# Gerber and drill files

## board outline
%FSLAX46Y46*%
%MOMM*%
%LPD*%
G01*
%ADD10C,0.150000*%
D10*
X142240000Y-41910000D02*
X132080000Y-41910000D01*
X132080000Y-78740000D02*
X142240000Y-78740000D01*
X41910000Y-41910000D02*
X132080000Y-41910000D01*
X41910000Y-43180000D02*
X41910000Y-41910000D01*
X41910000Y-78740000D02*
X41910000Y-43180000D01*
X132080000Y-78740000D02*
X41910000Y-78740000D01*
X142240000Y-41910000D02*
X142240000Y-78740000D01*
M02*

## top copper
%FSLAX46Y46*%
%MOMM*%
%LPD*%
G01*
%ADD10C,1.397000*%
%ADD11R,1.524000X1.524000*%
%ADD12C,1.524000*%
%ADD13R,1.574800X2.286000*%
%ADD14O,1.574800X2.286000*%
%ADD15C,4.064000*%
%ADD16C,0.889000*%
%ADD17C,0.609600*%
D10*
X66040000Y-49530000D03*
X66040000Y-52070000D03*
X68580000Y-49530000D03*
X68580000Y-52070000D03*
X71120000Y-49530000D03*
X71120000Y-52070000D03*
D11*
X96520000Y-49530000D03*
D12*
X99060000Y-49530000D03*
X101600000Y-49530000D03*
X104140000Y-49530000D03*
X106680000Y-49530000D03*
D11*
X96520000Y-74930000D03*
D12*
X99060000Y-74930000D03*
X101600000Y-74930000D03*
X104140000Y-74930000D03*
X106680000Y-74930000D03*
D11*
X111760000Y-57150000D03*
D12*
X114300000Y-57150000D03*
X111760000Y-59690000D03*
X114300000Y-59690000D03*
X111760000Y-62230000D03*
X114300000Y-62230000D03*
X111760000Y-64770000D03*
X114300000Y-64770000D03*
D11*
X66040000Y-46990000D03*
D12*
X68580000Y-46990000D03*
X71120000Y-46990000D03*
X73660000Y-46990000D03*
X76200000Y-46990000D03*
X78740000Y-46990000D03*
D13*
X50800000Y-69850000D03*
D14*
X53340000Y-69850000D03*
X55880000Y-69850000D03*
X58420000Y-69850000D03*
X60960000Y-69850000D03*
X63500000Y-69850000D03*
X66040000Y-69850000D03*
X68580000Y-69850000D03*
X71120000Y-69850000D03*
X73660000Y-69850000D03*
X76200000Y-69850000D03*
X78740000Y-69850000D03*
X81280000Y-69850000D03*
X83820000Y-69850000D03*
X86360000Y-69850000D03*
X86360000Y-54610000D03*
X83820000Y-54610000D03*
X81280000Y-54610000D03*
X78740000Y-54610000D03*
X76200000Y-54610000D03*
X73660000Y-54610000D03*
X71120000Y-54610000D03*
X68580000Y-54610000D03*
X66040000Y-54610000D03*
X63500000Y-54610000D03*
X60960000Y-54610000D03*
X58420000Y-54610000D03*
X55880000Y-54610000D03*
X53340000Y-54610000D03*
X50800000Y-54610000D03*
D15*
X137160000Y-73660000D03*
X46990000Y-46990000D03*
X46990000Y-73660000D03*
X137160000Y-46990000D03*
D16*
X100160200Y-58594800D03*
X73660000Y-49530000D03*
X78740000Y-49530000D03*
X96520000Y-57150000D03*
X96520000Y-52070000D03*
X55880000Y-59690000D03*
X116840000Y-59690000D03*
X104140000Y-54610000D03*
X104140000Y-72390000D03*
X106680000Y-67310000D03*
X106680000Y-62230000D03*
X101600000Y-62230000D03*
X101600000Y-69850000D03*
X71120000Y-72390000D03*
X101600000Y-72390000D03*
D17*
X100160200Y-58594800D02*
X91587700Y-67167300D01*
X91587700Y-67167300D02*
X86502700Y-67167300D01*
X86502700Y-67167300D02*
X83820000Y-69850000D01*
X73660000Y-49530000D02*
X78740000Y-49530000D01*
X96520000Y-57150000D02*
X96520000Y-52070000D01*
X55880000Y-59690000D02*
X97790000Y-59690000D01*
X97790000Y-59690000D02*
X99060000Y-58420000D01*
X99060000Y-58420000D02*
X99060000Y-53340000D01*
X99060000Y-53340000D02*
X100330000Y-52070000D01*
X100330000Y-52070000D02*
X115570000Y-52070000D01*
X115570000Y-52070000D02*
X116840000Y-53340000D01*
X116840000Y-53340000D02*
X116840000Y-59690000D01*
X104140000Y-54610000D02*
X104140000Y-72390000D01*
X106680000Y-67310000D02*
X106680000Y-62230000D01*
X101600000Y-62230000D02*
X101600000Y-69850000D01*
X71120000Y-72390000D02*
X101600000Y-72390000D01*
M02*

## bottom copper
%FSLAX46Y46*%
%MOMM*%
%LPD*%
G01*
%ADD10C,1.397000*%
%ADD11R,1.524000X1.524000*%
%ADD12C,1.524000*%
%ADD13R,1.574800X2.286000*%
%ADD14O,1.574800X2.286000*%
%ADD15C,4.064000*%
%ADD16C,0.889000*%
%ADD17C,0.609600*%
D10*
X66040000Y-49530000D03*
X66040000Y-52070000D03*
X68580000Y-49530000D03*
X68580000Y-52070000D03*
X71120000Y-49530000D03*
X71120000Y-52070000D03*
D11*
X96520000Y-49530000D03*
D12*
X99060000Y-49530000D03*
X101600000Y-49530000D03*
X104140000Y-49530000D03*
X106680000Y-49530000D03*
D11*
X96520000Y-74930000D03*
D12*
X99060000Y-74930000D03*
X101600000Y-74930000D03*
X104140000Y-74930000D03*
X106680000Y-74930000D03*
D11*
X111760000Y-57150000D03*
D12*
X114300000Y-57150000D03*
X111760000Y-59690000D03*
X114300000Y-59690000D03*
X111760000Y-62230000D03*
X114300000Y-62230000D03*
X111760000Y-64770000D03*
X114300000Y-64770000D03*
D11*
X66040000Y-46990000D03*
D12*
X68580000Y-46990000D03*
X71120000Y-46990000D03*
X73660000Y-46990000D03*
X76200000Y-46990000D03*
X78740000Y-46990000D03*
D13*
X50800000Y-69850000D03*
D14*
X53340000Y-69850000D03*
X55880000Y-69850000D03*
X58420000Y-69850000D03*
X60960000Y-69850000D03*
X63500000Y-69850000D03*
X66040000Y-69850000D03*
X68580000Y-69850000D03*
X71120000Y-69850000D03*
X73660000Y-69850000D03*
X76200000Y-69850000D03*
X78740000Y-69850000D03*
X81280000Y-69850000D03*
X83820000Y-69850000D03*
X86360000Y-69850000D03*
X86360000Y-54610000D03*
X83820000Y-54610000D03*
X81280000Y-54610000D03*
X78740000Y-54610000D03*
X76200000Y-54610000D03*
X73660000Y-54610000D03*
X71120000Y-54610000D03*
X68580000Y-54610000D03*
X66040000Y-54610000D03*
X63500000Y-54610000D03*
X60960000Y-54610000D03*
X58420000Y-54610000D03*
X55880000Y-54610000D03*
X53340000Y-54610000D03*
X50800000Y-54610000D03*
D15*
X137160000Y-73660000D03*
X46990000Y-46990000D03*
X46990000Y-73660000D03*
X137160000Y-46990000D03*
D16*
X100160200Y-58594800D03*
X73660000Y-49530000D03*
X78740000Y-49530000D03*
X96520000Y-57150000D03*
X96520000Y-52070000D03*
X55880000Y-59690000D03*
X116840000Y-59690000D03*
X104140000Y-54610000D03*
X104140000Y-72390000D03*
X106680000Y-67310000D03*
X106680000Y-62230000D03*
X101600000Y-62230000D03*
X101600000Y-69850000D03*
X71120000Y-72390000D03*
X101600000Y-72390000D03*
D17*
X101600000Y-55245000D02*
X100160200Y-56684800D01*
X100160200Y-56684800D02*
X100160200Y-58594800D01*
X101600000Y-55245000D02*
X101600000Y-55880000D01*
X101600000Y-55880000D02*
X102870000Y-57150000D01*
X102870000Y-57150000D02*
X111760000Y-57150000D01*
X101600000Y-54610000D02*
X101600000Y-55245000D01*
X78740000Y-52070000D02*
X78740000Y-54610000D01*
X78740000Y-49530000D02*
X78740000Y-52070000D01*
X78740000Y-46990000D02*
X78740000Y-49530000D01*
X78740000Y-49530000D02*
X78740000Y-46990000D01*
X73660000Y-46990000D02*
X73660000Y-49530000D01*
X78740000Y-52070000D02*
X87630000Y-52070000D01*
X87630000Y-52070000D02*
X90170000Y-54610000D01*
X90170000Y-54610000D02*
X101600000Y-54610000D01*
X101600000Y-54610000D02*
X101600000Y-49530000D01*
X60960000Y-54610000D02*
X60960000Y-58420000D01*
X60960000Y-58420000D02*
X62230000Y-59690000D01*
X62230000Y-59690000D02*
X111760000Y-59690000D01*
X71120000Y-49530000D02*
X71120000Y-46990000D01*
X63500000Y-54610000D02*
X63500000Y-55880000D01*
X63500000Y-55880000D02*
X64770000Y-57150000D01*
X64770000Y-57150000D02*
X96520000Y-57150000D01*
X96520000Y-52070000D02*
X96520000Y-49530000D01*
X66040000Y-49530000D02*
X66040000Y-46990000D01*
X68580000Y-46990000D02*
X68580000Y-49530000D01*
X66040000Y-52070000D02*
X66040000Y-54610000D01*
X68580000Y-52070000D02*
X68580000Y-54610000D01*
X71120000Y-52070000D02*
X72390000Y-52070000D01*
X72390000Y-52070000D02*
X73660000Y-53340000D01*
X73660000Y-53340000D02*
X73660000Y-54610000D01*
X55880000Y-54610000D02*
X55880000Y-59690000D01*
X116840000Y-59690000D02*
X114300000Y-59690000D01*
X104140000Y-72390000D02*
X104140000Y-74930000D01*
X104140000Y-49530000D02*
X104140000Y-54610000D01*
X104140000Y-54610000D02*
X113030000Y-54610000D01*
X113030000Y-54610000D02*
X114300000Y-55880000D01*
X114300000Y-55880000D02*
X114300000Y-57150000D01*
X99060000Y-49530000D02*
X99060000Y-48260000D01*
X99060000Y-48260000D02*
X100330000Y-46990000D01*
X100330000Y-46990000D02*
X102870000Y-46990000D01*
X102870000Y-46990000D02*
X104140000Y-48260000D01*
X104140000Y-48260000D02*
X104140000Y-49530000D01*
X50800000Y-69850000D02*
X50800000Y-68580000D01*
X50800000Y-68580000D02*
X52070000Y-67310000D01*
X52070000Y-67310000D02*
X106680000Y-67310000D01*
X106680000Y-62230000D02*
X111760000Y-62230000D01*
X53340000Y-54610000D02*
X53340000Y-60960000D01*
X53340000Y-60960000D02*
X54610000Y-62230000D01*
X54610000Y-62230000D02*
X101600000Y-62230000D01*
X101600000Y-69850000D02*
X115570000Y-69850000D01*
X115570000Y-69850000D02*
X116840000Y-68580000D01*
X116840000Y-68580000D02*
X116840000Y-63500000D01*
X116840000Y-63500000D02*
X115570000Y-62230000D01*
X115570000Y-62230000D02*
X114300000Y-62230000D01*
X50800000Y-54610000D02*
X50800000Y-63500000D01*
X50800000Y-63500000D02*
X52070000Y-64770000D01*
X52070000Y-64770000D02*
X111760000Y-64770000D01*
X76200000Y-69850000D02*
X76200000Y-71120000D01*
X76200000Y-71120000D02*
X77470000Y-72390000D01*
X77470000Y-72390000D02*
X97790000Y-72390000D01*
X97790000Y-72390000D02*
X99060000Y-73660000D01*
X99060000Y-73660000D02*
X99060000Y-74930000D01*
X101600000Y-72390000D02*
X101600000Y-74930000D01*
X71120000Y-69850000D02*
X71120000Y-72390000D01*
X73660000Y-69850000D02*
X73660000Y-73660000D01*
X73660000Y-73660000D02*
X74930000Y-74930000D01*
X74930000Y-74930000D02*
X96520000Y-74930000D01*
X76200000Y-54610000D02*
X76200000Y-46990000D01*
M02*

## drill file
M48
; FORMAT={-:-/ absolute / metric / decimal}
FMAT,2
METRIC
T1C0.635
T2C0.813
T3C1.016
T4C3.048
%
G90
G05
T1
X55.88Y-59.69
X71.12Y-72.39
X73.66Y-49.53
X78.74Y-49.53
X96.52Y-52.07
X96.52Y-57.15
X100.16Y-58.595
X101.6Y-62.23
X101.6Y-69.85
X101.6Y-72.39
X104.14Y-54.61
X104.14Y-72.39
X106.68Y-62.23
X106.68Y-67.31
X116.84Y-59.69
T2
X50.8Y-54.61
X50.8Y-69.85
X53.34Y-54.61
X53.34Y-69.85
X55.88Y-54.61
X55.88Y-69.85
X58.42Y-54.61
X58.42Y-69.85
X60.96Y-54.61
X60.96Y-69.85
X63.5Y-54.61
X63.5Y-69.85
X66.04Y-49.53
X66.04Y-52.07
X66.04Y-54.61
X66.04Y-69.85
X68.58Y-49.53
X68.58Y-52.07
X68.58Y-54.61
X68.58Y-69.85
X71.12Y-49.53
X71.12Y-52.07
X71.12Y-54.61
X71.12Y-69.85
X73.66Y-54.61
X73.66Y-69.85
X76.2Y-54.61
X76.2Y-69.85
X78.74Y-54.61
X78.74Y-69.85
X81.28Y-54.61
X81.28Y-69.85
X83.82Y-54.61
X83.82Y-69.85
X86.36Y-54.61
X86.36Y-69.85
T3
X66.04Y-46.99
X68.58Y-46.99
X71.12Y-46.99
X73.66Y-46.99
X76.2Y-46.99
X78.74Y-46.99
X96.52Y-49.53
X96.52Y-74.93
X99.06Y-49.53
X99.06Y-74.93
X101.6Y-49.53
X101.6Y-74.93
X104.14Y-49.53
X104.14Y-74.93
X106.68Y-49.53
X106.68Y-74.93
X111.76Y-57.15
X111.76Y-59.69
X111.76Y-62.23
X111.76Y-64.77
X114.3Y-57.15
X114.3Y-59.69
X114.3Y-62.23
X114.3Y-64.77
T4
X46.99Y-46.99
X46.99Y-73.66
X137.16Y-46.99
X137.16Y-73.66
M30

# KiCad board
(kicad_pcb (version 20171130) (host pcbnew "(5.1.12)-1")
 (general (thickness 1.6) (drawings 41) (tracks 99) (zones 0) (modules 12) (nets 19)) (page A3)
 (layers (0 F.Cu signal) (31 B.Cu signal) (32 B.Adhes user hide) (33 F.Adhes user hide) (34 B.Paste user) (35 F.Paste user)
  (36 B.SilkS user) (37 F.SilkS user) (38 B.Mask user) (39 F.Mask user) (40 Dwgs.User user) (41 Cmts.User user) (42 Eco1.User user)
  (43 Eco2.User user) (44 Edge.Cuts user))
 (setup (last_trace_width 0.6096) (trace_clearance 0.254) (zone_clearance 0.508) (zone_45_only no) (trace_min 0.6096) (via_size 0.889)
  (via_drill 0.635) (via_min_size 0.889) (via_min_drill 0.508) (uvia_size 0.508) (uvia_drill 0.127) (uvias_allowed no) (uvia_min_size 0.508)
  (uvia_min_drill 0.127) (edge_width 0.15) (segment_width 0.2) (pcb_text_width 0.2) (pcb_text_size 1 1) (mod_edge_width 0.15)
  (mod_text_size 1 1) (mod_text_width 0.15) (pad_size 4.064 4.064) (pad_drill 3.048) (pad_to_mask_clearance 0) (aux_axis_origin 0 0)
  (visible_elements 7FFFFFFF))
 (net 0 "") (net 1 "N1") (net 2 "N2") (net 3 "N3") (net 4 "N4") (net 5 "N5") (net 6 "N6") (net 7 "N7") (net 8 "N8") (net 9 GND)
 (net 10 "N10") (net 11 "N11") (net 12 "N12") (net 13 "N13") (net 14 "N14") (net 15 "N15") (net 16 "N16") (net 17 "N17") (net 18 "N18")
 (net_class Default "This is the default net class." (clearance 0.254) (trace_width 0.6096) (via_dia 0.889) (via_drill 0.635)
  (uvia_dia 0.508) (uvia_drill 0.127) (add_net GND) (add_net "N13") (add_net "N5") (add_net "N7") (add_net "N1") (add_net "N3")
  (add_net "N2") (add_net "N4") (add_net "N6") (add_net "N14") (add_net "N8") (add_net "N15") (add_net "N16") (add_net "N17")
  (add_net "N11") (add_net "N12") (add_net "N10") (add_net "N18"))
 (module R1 (layer F.Cu) (at 66.04 50.8 270) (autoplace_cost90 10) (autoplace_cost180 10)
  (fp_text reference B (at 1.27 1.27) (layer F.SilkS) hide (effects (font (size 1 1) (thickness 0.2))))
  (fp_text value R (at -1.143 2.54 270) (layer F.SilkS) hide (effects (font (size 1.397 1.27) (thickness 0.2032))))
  (pad 1 thru_hole circle (at -1.27 0 270) (size 1.397 1.397) (drill 0.8128) (layers *.Cu *.Mask F.SilkS) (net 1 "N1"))
  (pad 2 thru_hole circle (at 1.27 0 270) (size 1.397 1.397) (drill 0.8128) (layers *.Cu *.Mask F.SilkS) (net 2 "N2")))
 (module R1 (layer F.Cu) (at 68.58 50.8 270) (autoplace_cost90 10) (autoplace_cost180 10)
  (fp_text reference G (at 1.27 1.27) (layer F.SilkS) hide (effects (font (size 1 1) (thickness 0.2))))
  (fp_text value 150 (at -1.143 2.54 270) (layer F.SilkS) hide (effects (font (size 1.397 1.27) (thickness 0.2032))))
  (pad 1 thru_hole circle (at -1.27 0 270) (size 1.397 1.397) (drill 0.8128) (layers *.Cu *.Mask F.SilkS) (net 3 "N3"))
  (pad 2 thru_hole circle (at 1.27 0 270) (size 1.397 1.397) (drill 0.8128) (layers *.Cu *.Mask F.SilkS) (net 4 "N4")))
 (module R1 (layer F.Cu) (at 71.12 50.8 270) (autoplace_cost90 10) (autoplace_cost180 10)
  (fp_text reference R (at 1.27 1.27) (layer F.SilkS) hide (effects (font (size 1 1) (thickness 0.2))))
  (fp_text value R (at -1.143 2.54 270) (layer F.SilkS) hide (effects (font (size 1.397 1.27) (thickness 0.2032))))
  (pad 1 thru_hole circle (at -1.27 0 270) (size 1.397 1.397) (drill 0.8128) (layers *.Cu *.Mask F.SilkS) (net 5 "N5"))
  (pad 2 thru_hole circle (at 1.27 0 270) (size 1.397 1.397) (drill 0.8128) (layers *.Cu *.Mask F.SilkS) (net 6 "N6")))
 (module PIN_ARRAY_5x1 (layer F.Cu) (at 101.6 49.53)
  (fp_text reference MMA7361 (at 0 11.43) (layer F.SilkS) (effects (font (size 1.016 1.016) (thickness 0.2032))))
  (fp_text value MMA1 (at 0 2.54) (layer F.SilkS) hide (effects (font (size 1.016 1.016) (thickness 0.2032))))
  (pad 1 thru_hole rect (at -5.08 0) (size 1.524 1.524) (drill 1.016) (layers *.Cu *.Mask F.SilkS) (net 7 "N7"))
  (pad 2 thru_hole circle (at -2.54 0) (size 1.524 1.524) (drill 1.016) (layers *.Cu *.Mask F.SilkS) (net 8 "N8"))
  (pad 3 thru_hole circle (at 0 0) (size 1.524 1.524) (drill 1.016) (layers *.Cu *.Mask F.SilkS) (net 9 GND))
  (pad 4 thru_hole circle (at 2.54 0) (size 1.524 1.524) (drill 1.016) (layers *.Cu *.Mask F.SilkS) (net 8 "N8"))
  (pad 5 thru_hole circle (at 5.08 0) (size 1.524 1.524) (drill 1.016) (layers *.Cu *.Mask F.SilkS)))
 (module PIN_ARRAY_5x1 (layer F.Cu) (at 101.6 74.93)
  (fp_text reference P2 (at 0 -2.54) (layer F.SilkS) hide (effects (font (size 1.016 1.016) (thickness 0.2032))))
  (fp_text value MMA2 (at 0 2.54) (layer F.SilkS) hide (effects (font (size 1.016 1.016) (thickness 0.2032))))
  (pad 1 thru_hole rect (at -5.08 0) (size 1.524 1.524) (drill 1.016) (layers *.Cu *.Mask F.SilkS) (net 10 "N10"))
  (pad 2 thru_hole circle (at -2.54 0) (size 1.524 1.524) (drill 1.016) (layers *.Cu *.Mask F.SilkS) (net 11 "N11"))
  (pad 3 thru_hole circle (at 0 0) (size 1.524 1.524) (drill 1.016) (layers *.Cu *.Mask F.SilkS) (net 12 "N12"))
  (pad 4 thru_hole circle (at 2.54 0) (size 1.524 1.524) (drill 1.016) (layers *.Cu *.Mask F.SilkS) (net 8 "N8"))
  (pad 5 thru_hole circle (at 5.08 0) (size 1.524 1.524) (drill 1.016) (layers *.Cu *.Mask F.SilkS)))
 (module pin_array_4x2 (layer F.Cu) (at 113.03 60.96 270)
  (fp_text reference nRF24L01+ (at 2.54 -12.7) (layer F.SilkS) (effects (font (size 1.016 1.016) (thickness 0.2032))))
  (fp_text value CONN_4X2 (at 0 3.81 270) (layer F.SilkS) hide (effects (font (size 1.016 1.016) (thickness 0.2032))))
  (pad 1 thru_hole rect (at -3.81 1.27 270) (size 1.524 1.524) (drill 1.016) (layers *.Cu *.Mask F.SilkS) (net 9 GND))
  (pad 2 thru_hole circle (at -3.81 -1.27 270) (size 1.524 1.524) (drill 1.016) (layers *.Cu *.Mask F.SilkS) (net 8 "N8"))
  (pad 3 thru_hole circle (at -1.27 1.27 270) (size 1.524 1.524) (drill 1.016) (layers *.Cu *.Mask F.SilkS) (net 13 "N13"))
  (pad 4 thru_hole circle (at -1.27 -1.27 270) (size 1.524 1.524) (drill 1.016) (layers *.Cu *.Mask F.SilkS) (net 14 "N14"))
  (pad 5 thru_hole circle (at 1.27 1.27 270) (size 1.524 1.524) (drill 1.016) (layers *.Cu *.Mask F.SilkS) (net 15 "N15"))
  (pad 6 thru_hole circle (at 1.27 -1.27 270) (size 1.524 1.524) (drill 1.016) (layers *.Cu *.Mask F.SilkS) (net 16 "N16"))
  (pad 7 thru_hole circle (at 3.81 1.27 270) (size 1.524 1.524) (drill 1.016) (layers *.Cu *.Mask F.SilkS) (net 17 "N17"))
  (pad 8 thru_hole circle (at 3.81 -1.27 270) (size 1.524 1.524) (drill 1.016) (layers *.Cu *.Mask F.SilkS)))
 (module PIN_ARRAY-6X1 (layer F.Cu) (at 72.39 46.99)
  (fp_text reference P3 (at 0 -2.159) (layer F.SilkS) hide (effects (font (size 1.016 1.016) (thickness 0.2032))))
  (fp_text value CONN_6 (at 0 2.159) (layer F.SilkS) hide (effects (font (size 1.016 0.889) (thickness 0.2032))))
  (pad 1 thru_hole rect (at -6.35 0) (size 1.524 1.524) (drill 1.016) (layers *.Cu *.Mask F.SilkS) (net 1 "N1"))
  (pad 2 thru_hole circle (at -3.81 0) (size 1.524 1.524) (drill 1.016) (layers *.Cu *.Mask F.SilkS) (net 3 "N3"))
  (pad 3 thru_hole circle (at -1.27 0) (size 1.524 1.524) (drill 1.016) (layers *.Cu *.Mask F.SilkS) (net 5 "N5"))
  (pad 4 thru_hole circle (at 1.27 0) (size 1.524 1.524) (drill 1.016) (layers *.Cu *.Mask F.SilkS) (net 9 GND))
  (pad 5 thru_hole circle (at 3.81 0) (size 1.524 1.524) (drill 1.016) (layers *.Cu *.Mask F.SilkS) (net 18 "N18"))
  (pad 6 thru_hole circle (at 6.35 0) (size 1.524 1.524) (drill 1.016) (layers *.Cu *.Mask F.SilkS) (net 9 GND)))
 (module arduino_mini (layer F.Cu) (at 69.85 62.23)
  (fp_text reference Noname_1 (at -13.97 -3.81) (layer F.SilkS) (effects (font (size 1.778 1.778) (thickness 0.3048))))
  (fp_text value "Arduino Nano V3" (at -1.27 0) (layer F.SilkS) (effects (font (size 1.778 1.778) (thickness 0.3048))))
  (pad 1 thru_hole rect (at -19.05 7.62) (size 1.5748 2.286) (drill 0.8128) (layers *.Cu *.Mask F.SilkS) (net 15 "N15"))
  (pad 2 thru_hole oval (at -16.51 7.62) (size 1.5748 2.286) (drill 0.8128) (layers *.Cu *.Mask F.SilkS))
  (pad 3 thru_hole oval (at -13.97 7.62) (size 1.5748 2.286) (drill 0.8128) (layers *.Cu *.Mask F.SilkS))
  (pad 4 thru_hole oval (at -11.43 7.62) (size 1.5748 2.286) (drill 0.8128) (layers *.Cu *.Mask F.SilkS))
  (pad 5 thru_hole oval (at -8.89 7.62) (size 1.5748 2.286) (drill 0.8128) (layers *.Cu *.Mask F.SilkS))
  (pad 6 thru_hole oval (at -6.35 7.62) (size 1.5748 2.286) (drill 0.8128) (layers *.Cu *.Mask F.SilkS))
  (pad 7 thru_hole oval (at -3.81 7.62) (size 1.5748 2.286) (drill 0.8128) (layers *.Cu *.Mask F.SilkS))
  (pad 8 thru_hole oval (at -1.27 7.62) (size 1.5748 2.286) (drill 0.8128) (layers *.Cu *.Mask F.SilkS))
  (pad 9 thru_hole oval (at 1.27 7.62) (size 1.5748 2.286) (drill 0.8128) (layers *.Cu *.Mask F.SilkS) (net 12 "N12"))
  (pad 10 thru_hole oval (at 3.81 7.62) (size 1.5748 2.286) (drill 0.8128) (layers *.Cu *.Mask F.SilkS) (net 10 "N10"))
  (pad 11 thru_hole oval (at 6.35 7.62) (size 1.5748 2.286) (drill 0.8128) (layers *.Cu *.Mask F.SilkS) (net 11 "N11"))
  (pad 12 thru_hole oval (at 8.89 7.62) (size 1.5748 2.286) (drill 0.8128) (layers *.Cu *.Mask F.SilkS))
  (pad 13 thru_hole oval (at 11.43 7.62) (size 1.5748 2.286) (drill 0.8128) (layers *.Cu *.Mask F.SilkS))
  (pad 14 thru_hole oval (at 13.97 7.62) (size 1.5748 2.286) (drill 0.8128) (layers *.Cu *.Mask F.SilkS) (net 9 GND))
  (pad 15 thru_hole oval (at 16.51 7.62) (size 1.5748 2.286) (drill 0.8128) (layers *.Cu *.Mask F.SilkS))
  (pad 16 thru_hole oval (at 16.51 -7.62) (size 1.5748 2.286) (drill 0.8128) (layers *.Cu *.Mask F.SilkS))
  (pad 17 thru_hole oval (at 13.97 -7.62) (size 1.5748 2.286) (drill 0.8128) (layers *.Cu *.Mask F.SilkS))
  (pad 18 thru_hole oval (at 11.43 -7.62) (size 1.5748 2.286) (drill 0.8128) (layers *.Cu *.Mask F.SilkS))
  (pad 19 thru_hole oval (at 8.89 -7.62) (size 1.5748 2.286) (drill 0.8128) (layers *.Cu *.Mask F.SilkS) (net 9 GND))
  (pad 20 thru_hole oval (at 6.35 -7.62) (size 1.5748 2.286) (drill 0.8128) (layers *.Cu *.Mask F.SilkS) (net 18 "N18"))
  (pad 21 thru_hole oval (at 3.81 -7.62) (size 1.5748 2.286) (drill 0.8128) (layers *.Cu *.Mask F.SilkS) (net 6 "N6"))
  (pad 22 thru_hole oval (at 1.27 -7.62) (size 1.5748 2.286) (drill 0.8128) (layers *.Cu *.Mask F.SilkS))
  (pad 23 thru_hole oval (at -1.27 -7.62) (size 1.5748 2.286) (drill 0.8128) (layers *.Cu *.Mask F.SilkS) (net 4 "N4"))
  (pad 24 thru_hole oval (at -3.81 -7.62) (size 1.5748 2.286) (drill 0.8128) (layers *.Cu *.Mask F.SilkS) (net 2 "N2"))
  (pad 25 thru_hole oval (at -6.35 -7.62) (size 1.5748 2.286) (drill 0.8128) (layers *.Cu *.Mask F.SilkS) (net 7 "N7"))
  (pad 26 thru_hole oval (at -8.89 -7.62) (size 1.5748 2.286) (drill 0.8128) (layers *.Cu *.Mask F.SilkS) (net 13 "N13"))
  (pad 27 thru_hole oval (at -11.43 -7.62) (size 1.5748 2.286) (drill 0.8128) (layers *.Cu *.Mask F.SilkS))
  (pad 28 thru_hole oval (at -13.97 -7.62) (size 1.5748 2.286) (drill 0.8128) (layers *.Cu *.Mask F.SilkS) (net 14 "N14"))
  (pad 29 thru_hole oval (at -16.51 -7.62) (size 1.5748 2.286) (drill 0.8128) (layers *.Cu *.Mask F.SilkS) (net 16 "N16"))
  (pad 30 thru_hole oval (at -19.05 -7.62) (size 1.5748 2.286) (drill 0.8128) (layers *.Cu *.Mask F.SilkS) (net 17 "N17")))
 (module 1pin (layer F.Cu) (at 137.16 73.66)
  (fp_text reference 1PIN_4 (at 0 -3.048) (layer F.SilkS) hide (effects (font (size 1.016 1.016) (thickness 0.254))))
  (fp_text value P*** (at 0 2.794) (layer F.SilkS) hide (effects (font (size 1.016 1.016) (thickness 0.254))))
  (pad 1 thru_hole circle (at 0 0) (size 4.064 4.064) (drill 3.048) (layers *.Cu *.Mask F.SilkS)))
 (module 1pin (layer F.Cu) (at 46.99 46.99)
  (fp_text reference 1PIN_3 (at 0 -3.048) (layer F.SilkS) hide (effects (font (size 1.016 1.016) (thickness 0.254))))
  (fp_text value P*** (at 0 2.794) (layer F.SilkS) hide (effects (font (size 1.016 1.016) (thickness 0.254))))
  (pad 1 thru_hole circle (at 0 0) (size 4.064 4.064) (drill 3.048) (layers *.Cu *.Mask F.SilkS)))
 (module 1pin (layer F.Cu) (at 46.99 73.66)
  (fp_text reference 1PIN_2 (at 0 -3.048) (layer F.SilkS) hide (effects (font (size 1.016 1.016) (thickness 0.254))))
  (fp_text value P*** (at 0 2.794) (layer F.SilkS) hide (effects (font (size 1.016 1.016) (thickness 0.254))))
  (pad 1 thru_hole circle (at 0 0) (size 4.064 4.064) (drill 3.048) (layers *.Cu *.Mask F.SilkS)))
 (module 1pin (layer F.Cu) (at 137.16 46.99)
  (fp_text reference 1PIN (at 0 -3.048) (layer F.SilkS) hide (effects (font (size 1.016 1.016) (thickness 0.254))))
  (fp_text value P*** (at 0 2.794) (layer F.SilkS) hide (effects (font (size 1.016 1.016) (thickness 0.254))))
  (pad 1 thru_hole circle (at 0 0) (size 4.064 4.064) (drill 3.048) (layers *.Cu *.Mask F.SilkS)))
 (gr_line (start 142.24 41.91) (end 132.08 41.91) (angle 90) (layer Edge.Cuts) (width 0.15))
 (gr_line (start 132.08 78.74) (end 142.24 78.74) (angle 90) (layer Edge.Cuts) (width 0.15))
 (gr_line (start 41.91 41.91) (end 132.08 41.91) (angle 90) (layer Edge.Cuts) (width 0.15))
 (gr_line (start 41.91 43.18) (end 41.91 41.91) (angle 90) (layer Edge.Cuts) (width 0.15))
 (gr_line (start 41.91 78.74) (end 41.91 43.18) (angle 90) (layer Edge.Cuts) (width 0.15))
 (gr_line (start 132.08 78.74) (end 41.91 78.74) (angle 90) (layer Edge.Cuts) (width 0.15))
 (gr_line (start 142.24 41.91) (end 142.24 78.74) (angle 90) (layer Edge.Cuts) (width 0.15))
 (segment (start 100.1602 58.5948) (end 91.5877 67.1673) (width 0.6096) (layer F.Cu) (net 9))
 (segment (start 91.5877 67.1673) (end 86.5027 67.1673) (width 0.6096) (layer F.Cu) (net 9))
 (segment (start 86.5027 67.1673) (end 83.82 69.85) (width 0.6096) (layer F.Cu) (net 9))
 (segment (start 101.6 55.245) (end 100.1602 56.6848) (width 0.6096) (layer B.Cu) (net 9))
 (segment (start 100.1602 56.6848) (end 100.1602 58.5948) (width 0.6096) (layer B.Cu) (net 9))
 (segment (start 101.6 55.245) (end 101.6 55.88) (width 0.6096) (layer B.Cu) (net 9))
 (segment (start 101.6 55.88) (end 102.87 57.15) (width 0.6096) (layer B.Cu) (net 9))
 (segment (start 102.87 57.15) (end 111.76 57.15) (width 0.6096) (layer B.Cu) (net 9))
 (segment (start 101.6 54.61) (end 101.6 55.245) (width 0.6096) (layer B.Cu) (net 9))
 (segment (start 78.74 52.07) (end 78.74 54.61) (width 0.6096) (layer B.Cu) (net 9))
 (segment (start 78.74 49.53) (end 78.74 52.07) (width 0.6096) (layer B.Cu) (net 9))
 (segment (start 78.74 46.99) (end 78.74 49.53) (width 0.6096) (layer B.Cu) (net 9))
 (segment (start 73.66 49.53) (end 78.74 49.53) (width 0.6096) (layer F.Cu) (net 9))
 (segment (start 78.74 49.53) (end 78.74 46.99) (width 0.6096) (layer B.Cu) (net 9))
 (segment (start 73.66 46.99) (end 73.66 49.53) (width 0.6096) (layer B.Cu) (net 9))
 (segment (start 78.74 52.07) (end 87.63 52.07) (width 0.6096) (layer B.Cu) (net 9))
 (segment (start 87.63 52.07) (end 90.17 54.61) (width 0.6096) (layer B.Cu) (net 9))
 (segment (start 90.17 54.61) (end 101.6 54.61) (width 0.6096) (layer B.Cu) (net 9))
 (segment (start 101.6 54.61) (end 101.6 49.53) (width 0.6096) (layer B.Cu) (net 9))
 (via (at 100.1602 58.5948) (size 0.889) (layers F.Cu B.Cu) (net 9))
 (via (at 73.66 49.53) (size 0.889) (layers F.Cu B.Cu) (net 9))
 (via (at 78.74 49.53) (size 0.889) (layers F.Cu B.Cu) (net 9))
 (segment (start 60.96 54.61) (end 60.96 58.42) (width 0.6096) (layer B.Cu) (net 13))
 (segment (start 60.96 58.42) (end 62.23 59.69) (width 0.6096) (layer B.Cu) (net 13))
 (segment (start 62.23 59.69) (end 111.76 59.69) (width 0.6096) (layer B.Cu) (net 13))
 (segment (start 71.12 49.53) (end 71.12 46.99) (width 0.6096) (layer B.Cu) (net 5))
 (segment (start 63.5 54.61) (end 63.5 55.88) (width 0.6096) (layer B.Cu) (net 7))
 (segment (start 63.5 55.88) (end 64.77 57.15) (width 0.6096) (layer B.Cu) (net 7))
 (segment (start 64.77 57.15) (end 96.52 57.15) (width 0.6096) (layer B.Cu) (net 7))
 (segment (start 96.52 57.15) (end 96.52 52.07) (width 0.6096) (layer F.Cu) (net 7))
 (segment (start 96.52 52.07) (end 96.52 49.53) (width 0.6096) (layer B.Cu) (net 7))
 (via (at 96.52 57.15) (size 0.889) (layers F.Cu B.Cu) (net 7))
 (via (at 96.52 52.07) (size 0.889) (layers F.Cu B.Cu) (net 7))
 (segment (start 66.04 49.53) (end 66.04 46.99) (width 0.6096) (layer B.Cu) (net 1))
 (segment (start 68.58 46.99) (end 68.58 49.53) (width 0.6096) (layer B.Cu) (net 3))
 (segment (start 66.04 52.07) (end 66.04 54.61) (width 0.6096) (layer B.Cu) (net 2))
 (segment (start 68.58 52.07) (end 68.58 54.61) (width 0.6096) (layer B.Cu) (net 4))
 (segment (start 71.12 52.07) (end 72.39 52.07) (width 0.6096) (layer B.Cu) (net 6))
 (segment (start 72.39 52.07) (end 73.66 53.34) (width 0.6096) (layer B.Cu) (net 6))
 (segment (start 73.66 53.34) (end 73.66 54.61) (width 0.6096) (layer B.Cu) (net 6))
 (segment (start 55.88 54.61) (end 55.88 59.69) (width 0.6096) (layer B.Cu) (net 14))
 (segment (start 116.84 59.69) (end 114.3 59.69) (width 0.6096) (layer B.Cu) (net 14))
 (segment (start 55.88 59.69) (end 97.79 59.69) (width 0.6096) (layer F.Cu) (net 14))
 (segment (start 97.79 59.69) (end 99.06 58.42) (width 0.6096) (layer F.Cu) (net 14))
 (segment (start 99.06 58.42) (end 99.06 53.34) (width 0.6096) (layer F.Cu) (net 14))
 (segment (start 99.06 53.34) (end 100.33 52.07) (width 0.6096) (layer F.Cu) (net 14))
 (segment (start 100.33 52.07) (end 115.57 52.07) (width 0.6096) (layer F.Cu) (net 14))
 (segment (start 115.57 52.07) (end 116.84 53.34) (width 0.6096) (layer F.Cu) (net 14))
 (segment (start 116.84 53.34) (end 116.84 59.69) (width 0.6096) (layer F.Cu) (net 14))
 (via (at 55.88 59.69) (size 0.889) (layers F.Cu B.Cu) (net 14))
 (via (at 116.84 59.69) (size 0.889) (layers F.Cu B.Cu) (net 14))
 (segment (start 104.14 54.61) (end 104.14 72.39) (width 0.6096) (layer F.Cu) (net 8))
 (segment (start 104.14 72.39) (end 104.14 74.93) (width 0.6096) (layer B.Cu) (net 8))
 (segment (start 104.14 49.53) (end 104.14 54.61) (width 0.6096) (layer B.Cu) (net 8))
 (segment (start 104.14 54.61) (end 113.03 54.61) (width 0.6096) (layer B.Cu) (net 8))
 (segment (start 113.03 54.61) (end 114.3 55.88) (width 0.6096) (layer B.Cu) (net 8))
 (segment (start 114.3 55.88) (end 114.3 57.15) (width 0.6096) (layer B.Cu) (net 8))
 (segment (start 99.06 49.53) (end 99.06 48.26) (width 0.6096) (layer B.Cu) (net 8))
 (segment (start 99.06 48.26) (end 100.33 46.99) (width 0.6096) (layer B.Cu) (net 8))
 (segment (start 100.33 46.99) (end 102.87 46.99) (width 0.6096) (layer B.Cu) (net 8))
 (segment (start 102.87 46.99) (end 104.14 48.26) (width 0.6096) (layer B.Cu) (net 8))
 (segment (start 104.14 48.26) (end 104.14 49.53) (width 0.6096) (layer B.Cu) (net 8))
 (via (at 104.14 54.61) (size 0.889) (layers F.Cu B.Cu) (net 8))
 (via (at 104.14 72.39) (size 0.889) (layers F.Cu B.Cu) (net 8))
 (segment (start 50.8 69.85) (end 50.8 68.58) (width 0.6096) (layer B.Cu) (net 15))
 (segment (start 50.8 68.58) (end 52.07 67.31) (width 0.6096) (layer B.Cu) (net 15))
 (segment (start 52.07 67.31) (end 106.68 67.31) (width 0.6096) (layer B.Cu) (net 15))
 (segment (start 106.68 67.31) (end 106.68 62.23) (width 0.6096) (layer F.Cu) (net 15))
 (segment (start 106.68 62.23) (end 111.76 62.23) (width 0.6096) (layer B.Cu) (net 15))
 (via (at 106.68 67.31) (size 0.889) (layers F.Cu B.Cu) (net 15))
 (via (at 106.68 62.23) (size 0.889) (layers F.Cu B.Cu) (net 15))
 (segment (start 53.34 54.61) (end 53.34 60.96) (width 0.6096) (layer B.Cu) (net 16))
 (segment (start 53.34 60.96) (end 54.61 62.23) (width 0.6096) (layer B.Cu) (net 16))
 (segment (start 54.61 62.23) (end 101.6 62.23) (width 0.6096) (layer B.Cu) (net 16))
 (segment (start 101.6 62.23) (end 101.6 69.85) (width 0.6096) (layer F.Cu) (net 16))
 (segment (start 101.6 69.85) (end 115.57 69.85) (width 0.6096) (layer B.Cu) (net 16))
 (segment (start 115.57 69.85) (end 116.84 68.58) (width 0.6096) (layer B.Cu) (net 16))
 (segment (start 116.84 68.58) (end 116.84 63.5) (width 0.6096) (layer B.Cu) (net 16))
 (segment (start 116.84 63.5) (end 115.57 62.23) (width 0.6096) (layer B.Cu) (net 16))
 (segment (start 115.57 62.23) (end 114.3 62.23) (width 0.6096) (layer B.Cu) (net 16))
 (via (at 101.6 62.23) (size 0.889) (layers F.Cu B.Cu) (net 16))
 (via (at 101.6 69.85) (size 0.889) (layers F.Cu B.Cu) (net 16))
 (segment (start 50.8 54.61) (end 50.8 63.5) (width 0.6096) (layer B.Cu) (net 17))
 (segment (start 50.8 63.5) (end 52.07 64.77) (width 0.6096) (layer B.Cu) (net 17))
 (segment (start 52.07 64.77) (end 111.76 64.77) (width 0.6096) (layer B.Cu) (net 17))
 (segment (start 76.2 69.85) (end 76.2 71.12) (width 0.6096) (layer B.Cu) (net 11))
 (segment (start 76.2 71.12) (end 77.47 72.39) (width 0.6096) (layer B.Cu) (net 11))
 (segment (start 77.47 72.39) (end 97.79 72.39) (width 0.6096) (layer B.Cu) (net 11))
 (segment (start 97.79 72.39) (end 99.06 73.66) (width 0.6096) (layer B.Cu) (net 11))
 (segment (start 99.06 73.66) (end 99.06 74.93) (width 0.6096) (layer B.Cu) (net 11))
 (segment (start 71.12 72.39) (end 101.6 72.39) (width 0.6096) (layer F.Cu) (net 12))
 (segment (start 101.6 72.39) (end 101.6 74.93) (width 0.6096) (layer B.Cu) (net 12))
 (segment (start 71.12 69.85) (end 71.12 72.39) (width 0.6096) (layer B.Cu) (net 12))
 (via (at 71.12 72.39) (size 0.889) (layers F.Cu B.Cu) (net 12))
 (via (at 101.6 72.39) (size 0.889) (layers F.Cu B.Cu) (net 12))
 (segment (start 73.66 69.85) (end 73.66 73.66) (width 0.6096) (layer B.Cu) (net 10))
 (segment (start 73.66 73.66) (end 74.93 74.93) (width 0.6096) (layer B.Cu) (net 10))
 (segment (start 74.93 74.93) (end 96.52 74.93) (width 0.6096) (layer B.Cu) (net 10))
 (segment (start 76.2 54.61) (end 76.2 46.99) (width 0.6096) (layer B.Cu) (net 18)))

